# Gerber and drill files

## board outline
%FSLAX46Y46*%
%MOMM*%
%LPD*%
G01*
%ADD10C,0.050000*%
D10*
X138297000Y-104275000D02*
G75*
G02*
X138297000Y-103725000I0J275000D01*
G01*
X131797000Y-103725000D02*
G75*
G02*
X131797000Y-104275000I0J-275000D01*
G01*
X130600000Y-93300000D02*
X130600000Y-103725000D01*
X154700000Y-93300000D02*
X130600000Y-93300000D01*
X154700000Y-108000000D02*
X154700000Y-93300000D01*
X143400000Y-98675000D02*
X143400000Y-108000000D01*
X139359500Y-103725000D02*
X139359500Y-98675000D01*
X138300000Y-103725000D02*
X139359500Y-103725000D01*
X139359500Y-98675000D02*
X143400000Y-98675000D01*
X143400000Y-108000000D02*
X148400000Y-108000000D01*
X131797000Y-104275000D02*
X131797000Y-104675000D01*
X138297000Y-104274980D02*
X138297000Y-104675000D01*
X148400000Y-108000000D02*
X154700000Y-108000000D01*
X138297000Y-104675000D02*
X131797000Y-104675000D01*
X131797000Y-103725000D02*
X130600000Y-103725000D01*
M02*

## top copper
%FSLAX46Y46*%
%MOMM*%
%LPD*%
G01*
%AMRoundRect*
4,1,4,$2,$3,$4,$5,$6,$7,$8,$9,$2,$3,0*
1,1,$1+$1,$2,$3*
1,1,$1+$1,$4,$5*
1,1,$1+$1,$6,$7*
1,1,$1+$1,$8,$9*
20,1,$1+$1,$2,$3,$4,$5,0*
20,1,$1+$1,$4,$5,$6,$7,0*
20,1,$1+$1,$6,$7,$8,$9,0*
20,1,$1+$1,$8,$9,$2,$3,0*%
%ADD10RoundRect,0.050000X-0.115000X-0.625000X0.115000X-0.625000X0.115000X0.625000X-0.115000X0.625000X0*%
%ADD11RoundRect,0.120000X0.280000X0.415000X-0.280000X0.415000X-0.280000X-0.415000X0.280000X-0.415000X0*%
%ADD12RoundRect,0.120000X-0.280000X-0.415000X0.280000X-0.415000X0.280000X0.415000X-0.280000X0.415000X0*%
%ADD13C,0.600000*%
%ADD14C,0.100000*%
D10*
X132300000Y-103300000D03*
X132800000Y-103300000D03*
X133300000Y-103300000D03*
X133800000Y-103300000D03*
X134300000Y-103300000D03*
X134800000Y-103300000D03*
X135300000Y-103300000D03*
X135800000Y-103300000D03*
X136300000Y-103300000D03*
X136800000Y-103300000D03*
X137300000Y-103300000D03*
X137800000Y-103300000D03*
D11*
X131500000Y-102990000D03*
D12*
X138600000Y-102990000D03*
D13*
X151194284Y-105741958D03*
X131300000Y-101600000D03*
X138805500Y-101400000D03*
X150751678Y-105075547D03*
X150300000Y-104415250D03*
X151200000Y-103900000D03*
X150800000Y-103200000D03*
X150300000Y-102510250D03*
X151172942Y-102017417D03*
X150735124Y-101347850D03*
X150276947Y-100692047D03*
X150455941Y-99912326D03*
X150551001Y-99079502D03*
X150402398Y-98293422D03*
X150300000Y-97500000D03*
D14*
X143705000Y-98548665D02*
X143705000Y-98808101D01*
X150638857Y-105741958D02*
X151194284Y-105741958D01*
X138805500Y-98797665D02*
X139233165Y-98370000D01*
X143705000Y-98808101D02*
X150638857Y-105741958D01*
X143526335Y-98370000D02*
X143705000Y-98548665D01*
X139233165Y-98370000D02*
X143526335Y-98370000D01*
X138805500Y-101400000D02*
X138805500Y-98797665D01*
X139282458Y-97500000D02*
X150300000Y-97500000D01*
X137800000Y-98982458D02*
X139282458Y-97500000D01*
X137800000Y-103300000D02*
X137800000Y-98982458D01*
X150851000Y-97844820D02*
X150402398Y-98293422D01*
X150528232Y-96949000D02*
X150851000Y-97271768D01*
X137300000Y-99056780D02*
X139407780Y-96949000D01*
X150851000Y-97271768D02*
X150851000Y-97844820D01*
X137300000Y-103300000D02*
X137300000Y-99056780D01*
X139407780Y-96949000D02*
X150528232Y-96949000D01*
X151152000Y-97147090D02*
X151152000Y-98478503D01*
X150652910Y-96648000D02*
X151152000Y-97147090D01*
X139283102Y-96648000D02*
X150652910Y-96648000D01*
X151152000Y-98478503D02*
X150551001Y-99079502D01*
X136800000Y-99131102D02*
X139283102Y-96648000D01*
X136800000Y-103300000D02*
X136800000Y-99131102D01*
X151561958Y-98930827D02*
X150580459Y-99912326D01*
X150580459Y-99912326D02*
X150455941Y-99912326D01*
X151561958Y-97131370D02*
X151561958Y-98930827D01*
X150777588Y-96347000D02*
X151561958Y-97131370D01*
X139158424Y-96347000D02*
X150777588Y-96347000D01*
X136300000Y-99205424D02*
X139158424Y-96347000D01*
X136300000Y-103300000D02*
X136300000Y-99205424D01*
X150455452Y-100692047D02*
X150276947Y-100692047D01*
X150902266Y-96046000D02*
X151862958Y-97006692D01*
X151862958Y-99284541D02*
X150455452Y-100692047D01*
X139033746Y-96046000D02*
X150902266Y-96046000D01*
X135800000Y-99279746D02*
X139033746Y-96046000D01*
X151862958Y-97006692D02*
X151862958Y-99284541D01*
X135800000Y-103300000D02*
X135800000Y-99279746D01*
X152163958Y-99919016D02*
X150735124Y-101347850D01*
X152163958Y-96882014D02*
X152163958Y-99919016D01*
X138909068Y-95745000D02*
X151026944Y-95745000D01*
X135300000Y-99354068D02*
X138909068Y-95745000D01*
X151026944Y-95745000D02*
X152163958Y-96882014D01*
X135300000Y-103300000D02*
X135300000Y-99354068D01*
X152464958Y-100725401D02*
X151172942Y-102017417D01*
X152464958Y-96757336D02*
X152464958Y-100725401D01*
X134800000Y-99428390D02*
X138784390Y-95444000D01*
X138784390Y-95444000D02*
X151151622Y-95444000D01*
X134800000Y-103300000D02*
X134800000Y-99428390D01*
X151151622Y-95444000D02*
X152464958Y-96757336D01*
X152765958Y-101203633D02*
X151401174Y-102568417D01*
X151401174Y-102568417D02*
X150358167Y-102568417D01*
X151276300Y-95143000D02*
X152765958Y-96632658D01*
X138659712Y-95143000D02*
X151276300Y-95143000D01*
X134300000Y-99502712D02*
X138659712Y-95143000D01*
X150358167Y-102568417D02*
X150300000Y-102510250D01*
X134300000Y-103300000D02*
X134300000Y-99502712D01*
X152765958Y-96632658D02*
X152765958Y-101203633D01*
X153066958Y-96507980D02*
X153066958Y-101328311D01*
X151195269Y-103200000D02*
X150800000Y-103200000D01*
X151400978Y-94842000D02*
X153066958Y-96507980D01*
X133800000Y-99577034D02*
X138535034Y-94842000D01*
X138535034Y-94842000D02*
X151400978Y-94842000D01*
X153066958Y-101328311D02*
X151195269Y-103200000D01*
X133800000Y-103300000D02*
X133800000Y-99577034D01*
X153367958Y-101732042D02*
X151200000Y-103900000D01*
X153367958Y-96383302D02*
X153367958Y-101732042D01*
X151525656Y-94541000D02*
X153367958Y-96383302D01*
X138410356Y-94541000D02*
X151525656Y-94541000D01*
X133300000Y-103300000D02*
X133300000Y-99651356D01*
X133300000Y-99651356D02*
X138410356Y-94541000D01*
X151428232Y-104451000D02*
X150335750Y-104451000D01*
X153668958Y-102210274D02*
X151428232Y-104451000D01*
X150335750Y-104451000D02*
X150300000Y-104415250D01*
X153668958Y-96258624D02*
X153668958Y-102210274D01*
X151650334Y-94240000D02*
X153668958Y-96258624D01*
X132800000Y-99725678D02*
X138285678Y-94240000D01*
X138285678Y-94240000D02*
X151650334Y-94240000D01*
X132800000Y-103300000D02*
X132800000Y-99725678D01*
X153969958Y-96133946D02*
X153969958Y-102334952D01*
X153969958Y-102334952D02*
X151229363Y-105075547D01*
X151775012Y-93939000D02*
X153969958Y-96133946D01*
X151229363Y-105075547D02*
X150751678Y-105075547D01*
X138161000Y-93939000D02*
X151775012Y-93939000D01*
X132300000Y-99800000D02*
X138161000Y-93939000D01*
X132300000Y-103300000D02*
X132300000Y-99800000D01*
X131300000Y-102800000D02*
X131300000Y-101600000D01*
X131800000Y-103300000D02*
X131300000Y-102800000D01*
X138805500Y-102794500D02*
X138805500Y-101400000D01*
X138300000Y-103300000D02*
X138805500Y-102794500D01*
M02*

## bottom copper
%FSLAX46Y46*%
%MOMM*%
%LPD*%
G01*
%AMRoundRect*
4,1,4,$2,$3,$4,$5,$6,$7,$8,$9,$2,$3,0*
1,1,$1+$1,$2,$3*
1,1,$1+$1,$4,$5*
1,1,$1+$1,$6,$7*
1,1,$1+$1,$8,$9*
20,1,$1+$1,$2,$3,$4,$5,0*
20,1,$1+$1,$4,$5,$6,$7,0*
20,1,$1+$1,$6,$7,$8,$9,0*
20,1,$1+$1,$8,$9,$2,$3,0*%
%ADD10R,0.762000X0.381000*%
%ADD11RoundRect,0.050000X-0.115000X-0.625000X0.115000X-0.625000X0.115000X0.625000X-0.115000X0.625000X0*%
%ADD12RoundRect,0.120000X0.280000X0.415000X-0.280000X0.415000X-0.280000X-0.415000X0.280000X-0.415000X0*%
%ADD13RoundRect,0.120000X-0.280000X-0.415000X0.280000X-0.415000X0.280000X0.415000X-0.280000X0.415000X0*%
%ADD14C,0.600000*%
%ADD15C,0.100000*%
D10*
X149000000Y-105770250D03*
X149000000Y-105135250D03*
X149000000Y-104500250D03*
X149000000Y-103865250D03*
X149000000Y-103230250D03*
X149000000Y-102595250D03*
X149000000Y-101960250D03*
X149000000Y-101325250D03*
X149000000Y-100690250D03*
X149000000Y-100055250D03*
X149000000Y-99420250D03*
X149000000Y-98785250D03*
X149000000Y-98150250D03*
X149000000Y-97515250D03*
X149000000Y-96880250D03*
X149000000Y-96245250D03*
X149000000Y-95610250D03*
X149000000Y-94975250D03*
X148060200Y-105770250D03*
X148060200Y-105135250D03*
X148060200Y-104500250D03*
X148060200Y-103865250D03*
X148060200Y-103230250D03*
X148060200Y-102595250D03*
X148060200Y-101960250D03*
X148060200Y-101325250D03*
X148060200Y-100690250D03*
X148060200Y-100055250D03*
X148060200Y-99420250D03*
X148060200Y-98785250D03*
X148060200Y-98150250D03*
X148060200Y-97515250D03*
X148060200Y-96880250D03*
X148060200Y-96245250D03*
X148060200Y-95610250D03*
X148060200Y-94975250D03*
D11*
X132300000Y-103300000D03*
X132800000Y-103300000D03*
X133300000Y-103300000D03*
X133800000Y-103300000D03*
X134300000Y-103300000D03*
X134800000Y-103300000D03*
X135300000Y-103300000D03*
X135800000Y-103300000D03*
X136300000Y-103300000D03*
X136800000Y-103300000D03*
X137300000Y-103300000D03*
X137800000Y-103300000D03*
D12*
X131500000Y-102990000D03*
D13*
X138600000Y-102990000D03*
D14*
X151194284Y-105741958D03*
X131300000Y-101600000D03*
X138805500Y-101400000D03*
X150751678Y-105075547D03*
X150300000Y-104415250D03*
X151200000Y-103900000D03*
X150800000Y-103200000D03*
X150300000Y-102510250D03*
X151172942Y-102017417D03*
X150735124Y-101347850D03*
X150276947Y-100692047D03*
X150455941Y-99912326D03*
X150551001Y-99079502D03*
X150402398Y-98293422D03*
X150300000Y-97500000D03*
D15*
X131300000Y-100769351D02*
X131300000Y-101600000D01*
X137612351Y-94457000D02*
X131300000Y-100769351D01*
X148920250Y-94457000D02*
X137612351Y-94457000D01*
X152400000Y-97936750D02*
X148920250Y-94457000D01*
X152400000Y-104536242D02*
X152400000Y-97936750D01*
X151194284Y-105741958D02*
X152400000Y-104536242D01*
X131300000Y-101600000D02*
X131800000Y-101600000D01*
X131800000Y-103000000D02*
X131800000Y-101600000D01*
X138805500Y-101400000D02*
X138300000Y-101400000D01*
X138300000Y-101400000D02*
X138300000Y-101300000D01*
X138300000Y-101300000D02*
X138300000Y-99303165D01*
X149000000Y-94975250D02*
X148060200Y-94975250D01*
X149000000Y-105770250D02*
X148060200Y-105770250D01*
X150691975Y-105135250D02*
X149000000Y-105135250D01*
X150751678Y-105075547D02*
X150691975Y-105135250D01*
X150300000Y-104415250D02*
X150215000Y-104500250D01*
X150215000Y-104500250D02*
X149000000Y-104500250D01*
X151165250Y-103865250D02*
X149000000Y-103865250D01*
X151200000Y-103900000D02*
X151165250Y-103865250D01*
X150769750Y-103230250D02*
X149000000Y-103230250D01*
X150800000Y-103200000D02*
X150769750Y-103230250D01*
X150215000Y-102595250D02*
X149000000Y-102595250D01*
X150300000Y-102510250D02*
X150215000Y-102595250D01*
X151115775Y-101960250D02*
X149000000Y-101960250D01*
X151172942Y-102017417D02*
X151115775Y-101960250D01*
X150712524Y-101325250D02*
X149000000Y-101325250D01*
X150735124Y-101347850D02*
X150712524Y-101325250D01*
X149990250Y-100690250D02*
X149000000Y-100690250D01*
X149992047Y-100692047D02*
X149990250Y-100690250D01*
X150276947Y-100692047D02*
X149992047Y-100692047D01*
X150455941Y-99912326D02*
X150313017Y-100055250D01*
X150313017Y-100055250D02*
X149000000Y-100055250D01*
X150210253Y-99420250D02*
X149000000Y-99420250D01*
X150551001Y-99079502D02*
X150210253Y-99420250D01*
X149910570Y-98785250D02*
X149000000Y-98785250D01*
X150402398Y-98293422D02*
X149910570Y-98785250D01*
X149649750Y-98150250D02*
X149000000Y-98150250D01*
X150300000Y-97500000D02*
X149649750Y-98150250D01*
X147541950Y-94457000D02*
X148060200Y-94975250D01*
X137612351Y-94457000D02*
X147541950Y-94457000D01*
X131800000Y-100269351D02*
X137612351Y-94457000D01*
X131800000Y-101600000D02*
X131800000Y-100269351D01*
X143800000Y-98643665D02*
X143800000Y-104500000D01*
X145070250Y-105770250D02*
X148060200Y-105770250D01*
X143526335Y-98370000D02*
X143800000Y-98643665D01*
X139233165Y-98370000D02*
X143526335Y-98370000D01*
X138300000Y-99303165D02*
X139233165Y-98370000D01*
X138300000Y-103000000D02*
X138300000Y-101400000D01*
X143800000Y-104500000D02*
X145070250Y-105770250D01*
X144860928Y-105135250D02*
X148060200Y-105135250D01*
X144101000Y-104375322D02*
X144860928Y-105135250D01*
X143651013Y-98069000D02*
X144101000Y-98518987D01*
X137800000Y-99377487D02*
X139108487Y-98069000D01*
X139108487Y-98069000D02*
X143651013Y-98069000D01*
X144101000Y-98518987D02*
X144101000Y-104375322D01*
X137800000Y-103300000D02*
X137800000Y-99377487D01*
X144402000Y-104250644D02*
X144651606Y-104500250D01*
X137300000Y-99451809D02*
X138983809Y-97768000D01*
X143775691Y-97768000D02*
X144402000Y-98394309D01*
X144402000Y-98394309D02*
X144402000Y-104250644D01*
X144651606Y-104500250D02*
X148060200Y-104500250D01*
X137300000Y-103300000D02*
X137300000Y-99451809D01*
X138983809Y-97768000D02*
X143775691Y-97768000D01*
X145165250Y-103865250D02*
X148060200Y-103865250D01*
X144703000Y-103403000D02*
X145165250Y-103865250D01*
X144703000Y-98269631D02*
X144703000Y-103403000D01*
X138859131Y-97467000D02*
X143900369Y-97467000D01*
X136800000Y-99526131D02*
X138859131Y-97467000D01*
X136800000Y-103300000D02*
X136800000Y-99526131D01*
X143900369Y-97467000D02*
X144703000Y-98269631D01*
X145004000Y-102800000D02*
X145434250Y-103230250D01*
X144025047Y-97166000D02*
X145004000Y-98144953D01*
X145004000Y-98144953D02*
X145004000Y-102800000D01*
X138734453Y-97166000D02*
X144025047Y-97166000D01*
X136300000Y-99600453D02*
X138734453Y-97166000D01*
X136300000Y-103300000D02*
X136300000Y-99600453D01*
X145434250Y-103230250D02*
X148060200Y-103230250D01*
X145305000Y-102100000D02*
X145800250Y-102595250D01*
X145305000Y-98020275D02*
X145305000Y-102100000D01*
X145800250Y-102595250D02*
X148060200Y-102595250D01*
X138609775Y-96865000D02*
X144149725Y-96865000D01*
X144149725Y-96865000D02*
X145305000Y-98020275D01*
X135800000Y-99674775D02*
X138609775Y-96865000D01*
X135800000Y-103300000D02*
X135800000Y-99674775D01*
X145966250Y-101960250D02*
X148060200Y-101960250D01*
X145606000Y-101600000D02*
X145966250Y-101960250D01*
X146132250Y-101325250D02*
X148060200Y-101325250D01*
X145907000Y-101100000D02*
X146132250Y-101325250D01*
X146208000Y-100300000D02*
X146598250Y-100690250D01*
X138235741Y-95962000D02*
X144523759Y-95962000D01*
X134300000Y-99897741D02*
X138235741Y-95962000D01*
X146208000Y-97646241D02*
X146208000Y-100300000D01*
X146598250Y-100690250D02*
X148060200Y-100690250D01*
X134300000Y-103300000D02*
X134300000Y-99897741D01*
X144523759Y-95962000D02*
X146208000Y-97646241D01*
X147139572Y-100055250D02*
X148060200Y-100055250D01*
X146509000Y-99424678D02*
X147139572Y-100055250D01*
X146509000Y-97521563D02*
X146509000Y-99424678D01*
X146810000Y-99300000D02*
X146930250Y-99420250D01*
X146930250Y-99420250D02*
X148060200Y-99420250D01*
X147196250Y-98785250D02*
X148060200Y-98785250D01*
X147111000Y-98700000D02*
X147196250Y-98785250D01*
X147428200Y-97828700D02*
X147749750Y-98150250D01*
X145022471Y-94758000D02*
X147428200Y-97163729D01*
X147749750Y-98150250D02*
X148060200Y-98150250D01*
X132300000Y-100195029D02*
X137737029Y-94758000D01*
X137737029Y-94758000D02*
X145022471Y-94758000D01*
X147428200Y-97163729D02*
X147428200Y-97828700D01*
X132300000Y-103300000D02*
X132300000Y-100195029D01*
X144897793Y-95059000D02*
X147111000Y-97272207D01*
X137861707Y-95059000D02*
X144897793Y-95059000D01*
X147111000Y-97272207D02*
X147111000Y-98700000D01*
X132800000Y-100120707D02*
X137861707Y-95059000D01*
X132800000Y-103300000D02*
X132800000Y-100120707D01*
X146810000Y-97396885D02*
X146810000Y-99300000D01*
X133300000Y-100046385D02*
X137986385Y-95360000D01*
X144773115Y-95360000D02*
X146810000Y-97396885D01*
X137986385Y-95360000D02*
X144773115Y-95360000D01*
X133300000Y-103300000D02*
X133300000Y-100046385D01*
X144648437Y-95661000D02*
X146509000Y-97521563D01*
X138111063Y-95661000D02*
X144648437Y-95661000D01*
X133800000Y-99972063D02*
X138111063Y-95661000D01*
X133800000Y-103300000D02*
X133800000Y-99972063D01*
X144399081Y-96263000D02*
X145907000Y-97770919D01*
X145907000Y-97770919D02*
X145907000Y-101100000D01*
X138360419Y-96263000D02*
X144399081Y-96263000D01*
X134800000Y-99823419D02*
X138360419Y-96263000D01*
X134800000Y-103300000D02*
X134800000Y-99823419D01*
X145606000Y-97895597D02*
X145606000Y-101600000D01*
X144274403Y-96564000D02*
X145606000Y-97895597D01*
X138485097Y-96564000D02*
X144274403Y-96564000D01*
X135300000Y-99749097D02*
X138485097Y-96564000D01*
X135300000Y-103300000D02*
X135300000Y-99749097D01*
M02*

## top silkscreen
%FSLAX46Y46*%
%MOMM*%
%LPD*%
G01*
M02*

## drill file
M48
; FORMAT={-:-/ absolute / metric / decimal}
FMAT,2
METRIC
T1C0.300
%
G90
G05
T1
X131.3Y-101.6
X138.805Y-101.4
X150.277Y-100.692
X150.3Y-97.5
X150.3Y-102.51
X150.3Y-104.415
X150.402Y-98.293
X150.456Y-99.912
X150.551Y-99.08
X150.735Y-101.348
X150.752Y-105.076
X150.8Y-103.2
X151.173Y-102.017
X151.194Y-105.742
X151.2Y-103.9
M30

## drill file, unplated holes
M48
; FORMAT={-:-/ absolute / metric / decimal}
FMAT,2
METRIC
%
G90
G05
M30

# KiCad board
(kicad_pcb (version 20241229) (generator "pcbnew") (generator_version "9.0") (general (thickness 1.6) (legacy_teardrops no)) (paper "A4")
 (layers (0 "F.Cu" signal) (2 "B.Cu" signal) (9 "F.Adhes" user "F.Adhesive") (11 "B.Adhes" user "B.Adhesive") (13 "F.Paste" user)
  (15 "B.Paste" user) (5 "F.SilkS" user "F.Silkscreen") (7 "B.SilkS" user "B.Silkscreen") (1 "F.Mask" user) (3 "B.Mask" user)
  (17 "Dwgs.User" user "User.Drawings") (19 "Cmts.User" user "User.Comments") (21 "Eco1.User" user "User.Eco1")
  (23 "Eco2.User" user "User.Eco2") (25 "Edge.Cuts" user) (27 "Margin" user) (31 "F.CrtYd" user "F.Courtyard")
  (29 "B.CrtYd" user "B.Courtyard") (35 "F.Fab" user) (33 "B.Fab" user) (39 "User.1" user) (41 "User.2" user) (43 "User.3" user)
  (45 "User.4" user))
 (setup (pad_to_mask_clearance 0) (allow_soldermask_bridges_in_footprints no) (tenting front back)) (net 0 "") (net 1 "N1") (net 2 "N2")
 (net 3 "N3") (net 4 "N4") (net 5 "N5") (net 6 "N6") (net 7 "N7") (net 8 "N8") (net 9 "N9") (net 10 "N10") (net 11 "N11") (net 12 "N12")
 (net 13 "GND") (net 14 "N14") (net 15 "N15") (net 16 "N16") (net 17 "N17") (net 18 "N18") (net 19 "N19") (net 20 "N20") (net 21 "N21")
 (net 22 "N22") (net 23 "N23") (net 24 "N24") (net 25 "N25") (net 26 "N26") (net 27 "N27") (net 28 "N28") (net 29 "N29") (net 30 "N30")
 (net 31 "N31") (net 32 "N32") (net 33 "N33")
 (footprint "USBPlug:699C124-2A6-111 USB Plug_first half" (layer "F.Cu") (at 134.8 100.3)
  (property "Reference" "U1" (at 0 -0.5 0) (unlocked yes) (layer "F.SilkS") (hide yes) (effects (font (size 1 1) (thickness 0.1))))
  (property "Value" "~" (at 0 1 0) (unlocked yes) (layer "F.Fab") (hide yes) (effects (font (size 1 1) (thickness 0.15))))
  (pad "0" smd roundrect (at -2.5 3) (size 0.33 1.35) (layers "F.Cu" "F.Mask" "F.Paste") (roundrect_rratio 0.1515151515) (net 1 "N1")
   (thermal_bridge_angle 45))
  (pad "1" smd roundrect (at -2 3) (size 0.33 1.35) (layers "F.Cu" "F.Mask" "F.Paste") (roundrect_rratio 0.1515151515) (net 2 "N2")
   (thermal_bridge_angle 45))
  (pad "2" smd roundrect (at -1.5 3) (size 0.33 1.35) (layers "F.Cu" "F.Mask" "F.Paste") (roundrect_rratio 0.1515151515) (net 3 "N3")
   (thermal_bridge_angle 45))
  (pad "3" smd roundrect (at -1 3) (size 0.33 1.35) (layers "F.Cu" "F.Mask" "F.Paste") (roundrect_rratio 0.1515151515) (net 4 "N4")
   (thermal_bridge_angle 45))
  (pad "4" smd roundrect (at -0.5 3) (size 0.33 1.35) (layers "F.Cu" "F.Mask" "F.Paste") (roundrect_rratio 0.1515151515) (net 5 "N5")
   (thermal_bridge_angle 45))
  (pad "5" smd roundrect (at 0 3) (size 0.33 1.35) (layers "F.Cu" "F.Mask" "F.Paste") (roundrect_rratio 0.1515151515) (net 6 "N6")
   (thermal_bridge_angle 45))
  (pad "6" smd roundrect (at 0.5 3) (size 0.33 1.35) (layers "F.Cu" "F.Mask" "F.Paste") (roundrect_rratio 0.1515151515) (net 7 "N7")
   (thermal_bridge_angle 45))
  (pad "7" smd roundrect (at 1 3) (size 0.33 1.35) (layers "F.Cu" "F.Mask" "F.Paste") (roundrect_rratio 0.1515151515) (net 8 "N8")
   (thermal_bridge_angle 45))
  (pad "8" smd roundrect (at 1.5 3) (size 0.33 1.35) (layers "F.Cu" "F.Mask" "F.Paste") (roundrect_rratio 0.1515151515) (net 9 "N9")
   (thermal_bridge_angle 45))
  (pad "9" smd roundrect (at 2 3) (size 0.33 1.35) (layers "F.Cu" "F.Mask" "F.Paste") (roundrect_rratio 0.1515151515) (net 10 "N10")
   (thermal_bridge_angle 45))
  (pad "10" smd roundrect (at 2.5 3) (size 0.33 1.35) (layers "F.Cu" "F.Mask" "F.Paste") (roundrect_rratio 0.1515151515) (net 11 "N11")
   (thermal_bridge_angle 45))
  (pad "11" smd roundrect (at 3 3) (size 0.33 1.35) (layers "F.Cu" "F.Mask" "F.Paste") (roundrect_rratio 0.1515151515) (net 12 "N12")
   (thermal_bridge_angle 45))
  (pad "24" smd roundrect (at -3 3 180) (size 0.8 1.07) (drill (offset 0.3 0.31)) (layers "F.Cu" "F.Mask" "F.Paste") (roundrect_rratio 0.15)
   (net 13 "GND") (thermal_bridge_angle 45))
  (pad "25" smd roundrect (at 3.5 3) (size 0.8 1.07) (drill (offset 0.3 -0.31)) (layers "F.Cu" "F.Mask" "F.Paste") (roundrect_rratio 0.15)
   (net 13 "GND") (thermal_bridge_angle 45)))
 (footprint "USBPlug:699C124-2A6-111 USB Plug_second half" (layer "B.Cu") (at 134.8 106.3)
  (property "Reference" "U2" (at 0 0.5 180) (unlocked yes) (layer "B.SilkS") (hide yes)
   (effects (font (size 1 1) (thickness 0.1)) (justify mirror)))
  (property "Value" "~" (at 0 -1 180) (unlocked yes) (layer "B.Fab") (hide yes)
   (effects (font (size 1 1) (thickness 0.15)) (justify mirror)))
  (pad "12" smd roundrect (at -2.5 -3) (size 0.33 1.35) (layers "B.Cu" "B.Mask" "B.Paste") (roundrect_rratio 0.1515151515) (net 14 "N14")
   (thermal_bridge_angle 45))
  (pad "13" smd roundrect (at -2 -3) (size 0.33 1.35) (layers "B.Cu" "B.Mask" "B.Paste") (roundrect_rratio 0.1515151515) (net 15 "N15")
   (thermal_bridge_angle 45))
  (pad "14" smd roundrect (at -1.5 -3) (size 0.33 1.35) (layers "B.Cu" "B.Mask" "B.Paste") (roundrect_rratio 0.1515151515) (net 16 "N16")
   (thermal_bridge_angle 45))
  (pad "15" smd roundrect (at -1 -3) (size 0.33 1.35) (layers "B.Cu" "B.Mask" "B.Paste") (roundrect_rratio 0.1515151515) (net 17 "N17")
   (thermal_bridge_angle 45))
  (pad "16" smd roundrect (at -0.5 -3) (size 0.33 1.35) (layers "B.Cu" "B.Mask" "B.Paste") (roundrect_rratio 0.1515151515) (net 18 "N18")
   (thermal_bridge_angle 45))
  (pad "17" smd roundrect (at 0 -3) (size 0.33 1.35) (layers "B.Cu" "B.Mask" "B.Paste") (roundrect_rratio 0.1515151515) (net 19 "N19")
   (thermal_bridge_angle 45))
  (pad "18" smd roundrect (at 0.5 -3) (size 0.33 1.35) (layers "B.Cu" "B.Mask" "B.Paste") (roundrect_rratio 0.1515151515) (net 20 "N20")
   (thermal_bridge_angle 45))
  (pad "19" smd roundrect (at 1 -3) (size 0.33 1.35) (layers "B.Cu" "B.Mask" "B.Paste") (roundrect_rratio 0.1515151515) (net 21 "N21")
   (thermal_bridge_angle 45))
  (pad "20" smd roundrect (at 1.5 -3) (size 0.33 1.35) (layers "B.Cu" "B.Mask" "B.Paste") (roundrect_rratio 0.1515151515) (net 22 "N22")
   (thermal_bridge_angle 45))
  (pad "21" smd roundrect (at 2 -3) (size 0.33 1.35) (layers "B.Cu" "B.Mask" "B.Paste") (roundrect_rratio 0.1515151515) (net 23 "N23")
   (thermal_bridge_angle 45))
  (pad "22" smd roundrect (at 2.5 -3) (size 0.33 1.35) (layers "B.Cu" "B.Mask" "B.Paste") (roundrect_rratio 0.1515151515) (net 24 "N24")
   (thermal_bridge_angle 45))
  (pad "23" smd roundrect (at 3 -3) (size 0.33 1.35) (layers "B.Cu" "B.Mask" "B.Paste") (roundrect_rratio 0.1515151515) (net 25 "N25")
   (thermal_bridge_angle 45))
  (pad "26" smd roundrect (at -3 -3.3 180) (size 0.8 1.07) (drill (offset 0.3 0.01)) (layers "B.Cu" "B.Mask" "B.Paste")
   (roundrect_rratio 0.15) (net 13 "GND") (thermal_bridge_angle 45))
  (pad "27" smd roundrect (at 3.5 -3.3) (size 0.8 1.07) (drill (offset 0.3 -0.01)) (layers "B.Cu" "B.Mask" "B.Paste")
   (roundrect_rratio 0.15) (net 13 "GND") (thermal_bridge_angle 45)))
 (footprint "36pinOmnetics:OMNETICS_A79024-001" (layer "B.Cu") (at 148.5301 100.37275 -90)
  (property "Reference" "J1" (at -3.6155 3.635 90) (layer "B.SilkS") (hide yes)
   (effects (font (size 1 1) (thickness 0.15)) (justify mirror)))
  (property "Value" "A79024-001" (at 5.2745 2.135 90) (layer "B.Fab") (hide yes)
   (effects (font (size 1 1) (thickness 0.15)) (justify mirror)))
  (pad "1" smd rect (at 5.3975 -0.4699 270) (size 0.381 0.762) (layers "B.Cu" "B.Mask" "B.Paste") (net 13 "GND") (solder_mask_margin 0.102))
  (pad "2" smd rect (at 4.7625 -0.4699 270) (size 0.381 0.762) (layers "B.Cu" "B.Mask" "B.Paste") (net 1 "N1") (solder_mask_margin 0.102))
  (pad "3" smd rect (at 4.1275 -0.4699 270) (size 0.381 0.762) (layers "B.Cu" "B.Mask" "B.Paste") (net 2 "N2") (solder_mask_margin 0.102))
  (pad "4" smd rect (at 3.4925 -0.4699 270) (size 0.381 0.762) (layers "B.Cu" "B.Mask" "B.Paste") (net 3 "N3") (solder_mask_margin 0.102))
  (pad "5" smd rect (at 2.8575 -0.4699 270) (size 0.381 0.762) (layers "B.Cu" "B.Mask" "B.Paste") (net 4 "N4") (solder_mask_margin 0.102))
  (pad "6" smd rect (at 2.2225 -0.4699 270) (size 0.381 0.762) (layers "B.Cu" "B.Mask" "B.Paste") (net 5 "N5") (solder_mask_margin 0.102))
  (pad "7" smd rect (at 1.5875 -0.4699 270) (size 0.381 0.762) (layers "B.Cu" "B.Mask" "B.Paste") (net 6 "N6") (solder_mask_margin 0.102))
  (pad "8" smd rect (at 0.9525 -0.4699 270) (size 0.381 0.762) (layers "B.Cu" "B.Mask" "B.Paste") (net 7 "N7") (solder_mask_margin 0.102))
  (pad "9" smd rect (at 0.3175 -0.4699 270) (size 0.381 0.762) (layers "B.Cu" "B.Mask" "B.Paste") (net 8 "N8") (solder_mask_margin 0.102))
  (pad "10" smd rect (at -0.3175 -0.4699 270) (size 0.381 0.762) (layers "B.Cu" "B.Mask" "B.Paste") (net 9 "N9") (solder_mask_margin 0.102))
  (pad "11" smd rect (at -0.9525 -0.4699 270) (size 0.381 0.762) (layers "B.Cu" "B.Mask" "B.Paste") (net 10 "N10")
   (solder_mask_margin 0.102))
  (pad "12" smd rect (at -1.5875 -0.4699 270) (size 0.381 0.762) (layers "B.Cu" "B.Mask" "B.Paste") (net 11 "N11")
   (solder_mask_margin 0.102))
  (pad "13" smd rect (at -2.2225 -0.4699 270) (size 0.381 0.762) (layers "B.Cu" "B.Mask" "B.Paste") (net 12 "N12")
   (solder_mask_margin 0.102))
  (pad "14" smd rect (at -2.8575 -0.4699 270) (size 0.381 0.762) (layers "B.Cu" "B.Mask" "B.Paste") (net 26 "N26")
   (solder_mask_margin 0.102))
  (pad "15" smd rect (at -3.4925 -0.4699 270) (size 0.381 0.762) (layers "B.Cu" "B.Mask" "B.Paste") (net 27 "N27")
   (solder_mask_margin 0.102))
  (pad "16" smd rect (at -4.1275 -0.4699 270) (size 0.381 0.762) (layers "B.Cu" "B.Mask" "B.Paste") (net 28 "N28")
   (solder_mask_margin 0.102))
  (pad "17" smd rect (at -4.7625 -0.4699 270) (size 0.381 0.762) (layers "B.Cu" "B.Mask" "B.Paste") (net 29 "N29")
   (solder_mask_margin 0.102))
  (pad "18" smd rect (at -5.3975 -0.4699 270) (size 0.381 0.762) (layers "B.Cu" "B.Mask" "B.Paste") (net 13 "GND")
   (solder_mask_margin 0.102))
  (pad "19" smd rect (at 5.3975 0.4699 270) (size 0.381 0.762) (layers "B.Cu" "B.Mask" "B.Paste") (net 13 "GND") (solder_mask_margin 0.102))
  (pad "20" smd rect (at 4.7625 0.4699 270) (size 0.381 0.762) (layers "B.Cu" "B.Mask" "B.Paste") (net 25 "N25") (solder_mask_margin 0.102))
  (pad "21" smd rect (at 4.1275 0.4699 270) (size 0.381 0.762) (layers "B.Cu" "B.Mask" "B.Paste") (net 24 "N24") (solder_mask_margin 0.102))
  (pad "22" smd rect (at 3.4925 0.4699 270) (size 0.381 0.762) (layers "B.Cu" "B.Mask" "B.Paste") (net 23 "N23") (solder_mask_margin 0.102))
  (pad "23" smd rect (at 2.8575 0.4699 270) (size 0.381 0.762) (layers "B.Cu" "B.Mask" "B.Paste") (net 22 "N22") (solder_mask_margin 0.102))
  (pad "24" smd rect (at 2.2225 0.4699 270) (size 0.381 0.762) (layers "B.Cu" "B.Mask" "B.Paste") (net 21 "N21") (solder_mask_margin 0.102))
  (pad "25" smd rect (at 1.5875 0.4699 270) (size 0.381 0.762) (layers "B.Cu" "B.Mask" "B.Paste") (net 20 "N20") (solder_mask_margin 0.102))
  (pad "26" smd rect (at 0.9525 0.4699 270) (size 0.381 0.762) (layers "B.Cu" "B.Mask" "B.Paste") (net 19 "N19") (solder_mask_margin 0.102))
  (pad "27" smd rect (at 0.3175 0.4699 270) (size 0.381 0.762) (layers "B.Cu" "B.Mask" "B.Paste") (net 18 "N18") (solder_mask_margin 0.102))
  (pad "28" smd rect (at -0.3175 0.4699 270) (size 0.381 0.762) (layers "B.Cu" "B.Mask" "B.Paste") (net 17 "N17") (solder_mask_margin 0.102))
  (pad "29" smd rect (at -0.9525 0.4699 270) (size 0.381 0.762) (layers "B.Cu" "B.Mask" "B.Paste") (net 16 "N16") (solder_mask_margin 0.102))
  (pad "30" smd rect (at -1.5875 0.4699 270) (size 0.381 0.762) (layers "B.Cu" "B.Mask" "B.Paste") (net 15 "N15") (solder_mask_margin 0.102))
  (pad "31" smd rect (at -2.2225 0.4699 270) (size 0.381 0.762) (layers "B.Cu" "B.Mask" "B.Paste") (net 14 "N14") (solder_mask_margin 0.102))
  (pad "32" smd rect (at -2.8575 0.4699 270) (size 0.381 0.762) (layers "B.Cu" "B.Mask" "B.Paste") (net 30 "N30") (solder_mask_margin 0.102))
  (pad "33" smd rect (at -3.4925 0.4699 270) (size 0.381 0.762) (layers "B.Cu" "B.Mask" "B.Paste") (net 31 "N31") (solder_mask_margin 0.102))
  (pad "34" smd rect (at -4.1275 0.4699 270) (size 0.381 0.762) (layers "B.Cu" "B.Mask" "B.Paste") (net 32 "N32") (solder_mask_margin 0.102))
  (pad "35" smd rect (at -4.7625 0.4699 270) (size 0.381 0.762) (layers "B.Cu" "B.Mask" "B.Paste") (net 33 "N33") (solder_mask_margin 0.102))
  (pad "36" smd rect (at -5.3975 0.4699 270) (size 0.381 0.762) (layers "B.Cu" "B.Mask" "B.Paste") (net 13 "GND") (solder_mask_margin 0.102)))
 (gr_line (start 154.7 93.3) (end 130.6 93.3) (stroke (width 0.05) (type default)) (layer "Edge.Cuts"))
 (gr_line (start 130.6 93.3) (end 130.6 103.725) (stroke (width 0.05) (type default)) (layer "Edge.Cuts"))
 (gr_line (start 143.4 98.675) (end 143.4 108) (stroke (width 0.05) (type default)) (layer "Edge.Cuts"))
 (gr_line (start 139.3595 103.725) (end 139.3595 98.675) (stroke (width 0.05) (type default)) (layer "Edge.Cuts"))
 (gr_line (start 138.3 103.725) (end 139.3595 103.725) (stroke (width 0.05) (type default)) (layer "Edge.Cuts"))
 (gr_line (start 139.3595 98.675) (end 143.4 98.675) (stroke (width 0.05) (type default)) (layer "Edge.Cuts"))
 (gr_line (start 143.4 108) (end 148.4 108) (stroke (width 0.05) (type default)) (layer "Edge.Cuts"))
 (gr_line (start 131.797 104.275) (end 131.797 104.675) (stroke (width 0.05) (type default)) (layer "Edge.Cuts"))
 (gr_line (start 138.297 104.27498) (end 138.297 104.675) (stroke (width 0.05) (type default)) (layer "Edge.Cuts"))
 (gr_arc (start 131.797 103.725) (mid 132.072 104) (end 131.797 104.275) (stroke (width 0.05) (type default)) (layer "Edge.Cuts"))
 (gr_line (start 148.4 108) (end 154.7 108) (stroke (width 0.05) (type default)) (layer "Edge.Cuts"))
 (gr_arc (start 138.297 104.275) (mid 138.022 104) (end 138.297 103.725) (stroke (width 0.05) (type default)) (layer "Edge.Cuts"))
 (gr_line (start 154.7 108) (end 154.7 93.3) (stroke (width 0.05) (type default)) (layer "Edge.Cuts"))
 (gr_line (start 138.297 104.675) (end 131.797 104.675) (stroke (width 0.05) (type default)) (layer "Edge.Cuts"))
 (gr_line (start 131.797 103.725) (end 130.6 103.725) (stroke (width 0.05) (type default)) (layer "Edge.Cuts"))
 (segment (start 143.705 98.808101) (end 150.638857 105.741958) (width 0.1) (layer "F.Cu") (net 13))
 (segment (start 138.3 103.3) (end 138.8055 102.7945) (width 0.1) (layer "F.Cu") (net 13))
 (segment (start 131.3 102.8) (end 131.3 101.6) (width 0.1) (layer "F.Cu") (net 13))
 (segment (start 138.8055 101.4) (end 138.8055 98.797665) (width 0.1) (layer "F.Cu") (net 13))
 (segment (start 150.638857 105.741958) (end 151.194284 105.741958) (width 0.1) (layer "F.Cu") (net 13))
 (segment (start 138.8055 102.7945) (end 138.8055 101.4) (width 0.1) (layer "F.Cu") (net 13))
 (segment (start 138.8055 98.797665) (end 139.233165 98.37) (width 0.1) (layer "F.Cu") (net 13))
 (segment (start 139.233165 98.37) (end 143.526335 98.37) (width 0.1) (layer "F.Cu") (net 13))
 (segment (start 143.526335 98.37) (end 143.705 98.548665) (width 0.1) (layer "F.Cu") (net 13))
 (segment (start 143.705 98.548665) (end 143.705 98.808101) (width 0.1) (layer "F.Cu") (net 13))
 (segment (start 131.8 103.3) (end 131.3 102.8) (width 0.1) (layer "F.Cu") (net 13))
 (via (at 131.3 101.6) (size 0.6) (drill 0.3) (layers "F.Cu" "B.Cu") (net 13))
 (via (at 138.8055 101.4) (size 0.6) (drill 0.3) (layers "F.Cu" "B.Cu") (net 13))
 (via (at 151.194284 105.741958) (size 0.6) (drill 0.3) (layers "F.Cu" "B.Cu") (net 13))
 (segment (start 148.92025 94.457) (end 137.612351 94.457) (width 0.1) (layer "B.Cu") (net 13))
 (segment (start 145.07025 105.77025) (end 148.0602 105.77025) (width 0.1) (layer "B.Cu") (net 13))
 (segment (start 138.3 101.3) (end 138.3 99.303165) (width 0.1) (layer "B.Cu") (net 13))
 (segment (start 131.8 101.6) (end 131.8 100.269351) (width 0.1) (layer "B.Cu") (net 13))
 (segment (start 152.4 97.93675) (end 148.92025 94.457) (width 0.1) (layer "B.Cu") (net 13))
 (segment (start 143.526335 98.37) (end 143.8 98.643665) (width 0.1) (layer "B.Cu") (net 13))
 (segment (start 143.8 104.5) (end 145.07025 105.77025) (width 0.1) (layer "B.Cu") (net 13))
 (segment (start 139.233165 98.37) (end 143.526335 98.37) (width 0.1) (layer "B.Cu") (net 13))
 (segment (start 138.8055 101.4) (end 138.3 101.4) (width 0.1) (layer "B.Cu") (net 13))
 (segment (start 151.194284 105.741958) (end 152.4 104.536242) (width 0.1) (layer "B.Cu") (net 13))
 (segment (start 143.8 98.643665) (end 143.8 104.5) (width 0.1) (layer "B.Cu") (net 13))
 (segment (start 147.54195 94.457) (end 148.0602 94.97525) (width 0.1) (layer "B.Cu") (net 13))
 (segment (start 137.612351 94.457) (end 147.54195 94.457) (width 0.1) (layer "B.Cu") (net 13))
 (segment (start 149 105.77025) (end 148.0602 105.77025) (width 0.1) (layer "B.Cu") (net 13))
 (segment (start 138.3 103) (end 138.3 101.4) (width 0.1) (layer "B.Cu") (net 13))
 (segment (start 131.8 103) (end 131.8 101.6) (width 0.1) (layer "B.Cu") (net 13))
 (segment (start 131.3 100.769351) (end 131.3 101.6) (width 0.1) (layer "B.Cu") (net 13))
 (segment (start 137.612351 94.457) (end 131.3 100.769351) (width 0.1) (layer "B.Cu") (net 13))
 (segment (start 152.4 104.536242) (end 152.4 97.93675) (width 0.1) (layer "B.Cu") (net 13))
 (segment (start 149 94.97525) (end 148.0602 94.97525) (width 0.1) (layer "B.Cu") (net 13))
 (segment (start 131.3 101.6) (end 131.8 101.6) (width 0.1) (layer "B.Cu") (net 13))
 (segment (start 138.3 99.303165) (end 139.233165 98.37) (width 0.1) (layer "B.Cu") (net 13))
 (segment (start 138.3 101.4) (end 138.3 101.3) (width 0.1) (layer "B.Cu") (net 13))
 (segment (start 131.8 100.269351) (end 137.612351 94.457) (width 0.1) (layer "B.Cu") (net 13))
 (segment (start 133.3 99.651356) (end 138.410356 94.541) (width 0.1) (layer "F.Cu") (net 3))
 (segment (start 151.525656 94.541) (end 153.367958 96.383302) (width 0.1) (layer "F.Cu") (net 3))
 (segment (start 138.410356 94.541) (end 151.525656 94.541) (width 0.1) (layer "F.Cu") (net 3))
 (segment (start 153.367958 96.383302) (end 153.367958 101.732042) (width 0.1) (layer "F.Cu") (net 3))
 (segment (start 133.3 103.3) (end 133.3 99.651356) (width 0.1) (layer "F.Cu") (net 3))
 (segment (start 153.367958 101.732042) (end 151.2 103.9) (width 0.1) (layer "F.Cu") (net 3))
 (via (at 151.2 103.9) (size 0.6) (drill 0.3) (layers "F.Cu" "B.Cu") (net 3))
 (segment (start 151.2 103.9) (end 151.16525 103.86525) (width 0.1) (layer "B.Cu") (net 3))
 (segment (start 151.16525 103.86525) (end 149 103.86525) (width 0.1) (layer "B.Cu") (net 3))
 (segment (start 151.152 97.14709) (end 151.152 98.478503) (width 0.1) (layer "F.Cu") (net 10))
 (segment (start 136.8 103.3) (end 136.8 99.131102) (width 0.1) (layer "F.Cu") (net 10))
 (segment (start 139.283102 96.648) (end 150.65291 96.648) (width 0.1) (layer "F.Cu") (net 10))
 (segment (start 151.152 98.478503) (end 150.551001 99.079502) (width 0.1) (layer "F.Cu") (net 10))
 (segment (start 150.65291 96.648) (end 151.152 97.14709) (width 0.1) (layer "F.Cu") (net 10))
 (segment (start 136.8 99.131102) (end 139.283102 96.648) (width 0.1) (layer "F.Cu") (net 10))
 (via (at 150.551001 99.079502) (size 0.6) (drill 0.3) (layers "F.Cu" "B.Cu") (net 10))
 (segment (start 150.210253 99.42025) (end 149 99.42025) (width 0.1) (layer "B.Cu") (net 10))
 (segment (start 150.551001 99.079502) (end 150.210253 99.42025) (width 0.1) (layer "B.Cu") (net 10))
 (segment (start 152.765958 101.203633) (end 151.401174 102.568417) (width 0.1) (layer "F.Cu") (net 5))
 (segment (start 150.358167 102.568417) (end 150.3 102.51025) (width 0.1) (layer "F.Cu") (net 5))
 (segment (start 134.3 103.3) (end 134.3 99.502712) (width 0.1) (layer "F.Cu") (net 5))
 (segment (start 152.765958 96.632658) (end 152.765958 101.203633) (width 0.1) (layer "F.Cu") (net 5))
 (segment (start 134.3 99.502712) (end 138.659712 95.143) (width 0.1) (layer "F.Cu") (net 5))
 (segment (start 151.401174 102.568417) (end 150.358167 102.568417) (width 0.1) (layer "F.Cu") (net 5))
 (segment (start 151.2763 95.143) (end 152.765958 96.632658) (width 0.1) (layer "F.Cu") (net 5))
 (segment (start 138.659712 95.143) (end 151.2763 95.143) (width 0.1) (layer "F.Cu") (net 5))
 (via (at 150.3 102.51025) (size 0.6) (drill 0.3) (layers "F.Cu" "B.Cu") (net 5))
 (segment (start 150.3 102.51025) (end 150.215 102.59525) (width 0.1) (layer "B.Cu") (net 5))
 (segment (start 150.215 102.59525) (end 149 102.59525) (width 0.1) (layer "B.Cu") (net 5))
 (segment (start 139.033746 96.046) (end 150.902266 96.046) (width 0.1) (layer "F.Cu") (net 8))
 (segment (start 135.8 103.3) (end 135.8 99.279746) (width 0.1) (layer "F.Cu") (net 8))
 (segment (start 150.902266 96.046) (end 151.862958 97.006692) (width 0.1) (layer "F.Cu") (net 8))
 (segment (start 150.455452 100.692047) (end 150.276947 100.692047) (width 0.1) (layer "F.Cu") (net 8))
 (segment (start 135.8 99.279746) (end 139.033746 96.046) (width 0.1) (layer "F.Cu") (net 8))
 (segment (start 151.862958 97.006692) (end 151.862958 99.284541) (width 0.1) (layer "F.Cu") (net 8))
 (segment (start 151.862958 99.284541) (end 150.455452 100.692047) (width 0.1) (layer "F.Cu") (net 8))
 (via (at 150.276947 100.692047) (size 0.6) (drill 0.3) (layers "F.Cu" "B.Cu") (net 8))
 (segment (start 149.992047 100.692047) (end 149.99025 100.69025) (width 0.1) (layer "B.Cu") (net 8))
 (segment (start 149.99025 100.69025) (end 149 100.69025) (width 0.1) (layer "B.Cu") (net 8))
 (segment (start 150.276947 100.692047) (end 149.992047 100.692047) (width 0.1) (layer "B.Cu") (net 8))
 (segment (start 145.305 98.020275) (end 145.305 102.1) (width 0.1) (layer "B.Cu") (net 21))
 (segment (start 145.80025 102.59525) (end 148.0602 102.59525) (width 0.1) (layer "B.Cu") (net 21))
 (segment (start 135.8 99.674775) (end 138.609775 96.865) (width 0.1) (layer "B.Cu") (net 21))
 (segment (start 145.305 102.1) (end 145.80025 102.59525) (width 0.1) (layer "B.Cu") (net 21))
 (segment (start 144.149725 96.865) (end 145.305 98.020275) (width 0.1) (layer "B.Cu") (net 21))
 (segment (start 135.8 103.3) (end 135.8 99.674775) (width 0.1) (layer "B.Cu") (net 21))
 (segment (start 138.609775 96.865) (end 144.149725 96.865) (width 0.1) (layer "B.Cu") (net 21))
 (segment (start 145.004 102.8) (end 145.43425 103.23025) (width 0.1) (layer "B.Cu") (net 22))
 (segment (start 136.3 103.3) (end 136.3 99.600453) (width 0.1) (layer "B.Cu") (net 22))
 (segment (start 138.734453 97.166) (end 144.025047 97.166) (width 0.1) (layer "B.Cu") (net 22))
 (segment (start 136.3 99.600453) (end 138.734453 97.166) (width 0.1) (layer "B.Cu") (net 22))
 (segment (start 144.025047 97.166) (end 145.004 98.144953) (width 0.1) (layer "B.Cu") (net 22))
 (segment (start 145.43425 103.23025) (end 148.0602 103.23025) (width 0.1) (layer "B.Cu") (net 22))
 (segment (start 145.004 98.144953) (end 145.004 102.8) (width 0.1) (layer "B.Cu") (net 22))
 (segment (start 137.3 99.05678) (end 139.40778 96.949) (width 0.1) (layer "F.Cu") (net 11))
 (segment (start 150.528232 96.949) (end 150.851 97.271768) (width 0.1) (layer "F.Cu") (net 11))
 (segment (start 139.40778 96.949) (end 150.528232 96.949) (width 0.1) (layer "F.Cu") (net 11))
 (segment (start 150.851 97.271768) (end 150.851 97.84482) (width 0.1) (layer "F.Cu") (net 11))
 (segment (start 150.851 97.84482) (end 150.402398 98.293422) (width 0.1) (layer "F.Cu") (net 11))
 (segment (start 137.3 103.3) (end 137.3 99.05678) (width 0.1) (layer "F.Cu") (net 11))
 (via (at 150.402398 98.293422) (size 0.6) (drill 0.3) (layers "F.Cu" "B.Cu") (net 11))
 (segment (start 150.402398 98.293422) (end 149.91057 98.78525) (width 0.1) (layer "B.Cu") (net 11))
 (segment (start 149.91057 98.78525) (end 149 98.78525) (width 0.1) (layer "B.Cu") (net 11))
 (segment (start 152.464958 96.757336) (end 152.464958 100.725401) (width 0.1) (layer "F.Cu") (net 6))
 (segment (start 151.151622 95.444) (end 152.464958 96.757336) (width 0.1) (layer "F.Cu") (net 6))
 (segment (start 138.78439 95.444) (end 151.151622 95.444) (width 0.1) (layer "F.Cu") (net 6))
 (segment (start 134.8 99.42839) (end 138.78439 95.444) (width 0.1) (layer "F.Cu") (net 6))
 (segment (start 134.8 103.3) (end 134.8 99.42839) (width 0.1) (layer "F.Cu") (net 6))
 (segment (start 152.464958 100.725401) (end 151.172942 102.017417) (width 0.1) (layer "F.Cu") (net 6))
 (via (at 151.172942 102.017417) (size 0.6) (drill 0.3) (layers "F.Cu" "B.Cu") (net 6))
 (segment (start 151.172942 102.017417) (end 151.115775 101.96025) (width 0.1) (layer "B.Cu") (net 6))
 (segment (start 151.115775 101.96025) (end 149 101.96025) (width 0.1) (layer "B.Cu") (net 6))
 (segment (start 150.580459 99.912326) (end 150.455941 99.912326) (width 0.1) (layer "F.Cu") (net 9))
 (segment (start 151.561958 98.930827) (end 150.580459 99.912326) (width 0.1) (layer "F.Cu") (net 9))
 (segment (start 139.158424 96.347) (end 150.777588 96.347) (width 0.1) (layer "F.Cu") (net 9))
 (segment (start 136.3 99.205424) (end 139.158424 96.347) (width 0.1) (layer "F.Cu") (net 9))
 (segment (start 136.3 103.3) (end 136.3 99.205424) (width 0.1) (layer "F.Cu") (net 9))
 (segment (start 151.561958 97.13137) (end 151.561958 98.930827) (width 0.1) (layer "F.Cu") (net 9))
 (segment (start 150.777588 96.347) (end 151.561958 97.13137) (width 0.1) (layer "F.Cu") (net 9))
 (via (at 150.455941 99.912326) (size 0.6) (drill 0.3) (layers "F.Cu" "B.Cu") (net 9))
 (segment (start 150.455941 99.912326) (end 150.313017 100.05525) (width 0.1) (layer "B.Cu") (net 9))
 (segment (start 150.313017 100.05525) (end 149 100.05525) (width 0.1) (layer "B.Cu") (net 9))
 (segment (start 132.8 103.3) (end 132.8 99.725678) (width 0.1) (layer "F.Cu") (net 2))
 (segment (start 132.8 99.725678) (end 138.285678 94.24) (width 0.1) (layer "F.Cu") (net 2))
 (segment (start 151.428232 104.451) (end 150.33575 104.451) (width 0.1) (layer "F.Cu") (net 2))
 (segment (start 150.33575 104.451) (end 150.3 104.41525) (width 0.1) (layer "F.Cu") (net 2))
 (segment (start 153.668958 96.258624) (end 153.668958 102.210274) (width 0.1) (layer "F.Cu") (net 2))
 (segment (start 151.650334 94.24) (end 153.668958 96.258624) (width 0.1) (layer "F.Cu") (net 2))
 (segment (start 138.285678 94.24) (end 151.650334 94.24) (width 0.1) (layer "F.Cu") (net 2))
 (segment (start 153.668958 102.210274) (end 151.428232 104.451) (width 0.1) (layer "F.Cu") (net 2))
 (via (at 150.3 104.41525) (size 0.6) (drill 0.3) (layers "F.Cu" "B.Cu") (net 2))
 (segment (start 150.215 104.50025) (end 149 104.50025) (width 0.1) (layer "B.Cu") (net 2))
 (segment (start 150.3 104.41525) (end 150.215 104.50025) (width 0.1) (layer "B.Cu") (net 2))
 (segment (start 137.8 98.982458) (end 139.282458 97.5) (width 0.1) (layer "F.Cu") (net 12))
 (segment (start 137.8 103.3) (end 137.8 98.982458) (width 0.1) (layer "F.Cu") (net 12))
 (segment (start 139.282458 97.5) (end 150.3 97.5) (width 0.1) (layer "F.Cu") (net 12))
 (via (at 150.3 97.5) (size 0.6) (drill 0.3) (layers "F.Cu" "B.Cu") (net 12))
 (segment (start 149.64975 98.15025) (end 149 98.15025) (width 0.1) (layer "B.Cu") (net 12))
 (segment (start 150.3 97.5) (end 149.64975 98.15025) (width 0.1) (layer "B.Cu") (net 12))
 (segment (start 145.022471 94.758) (end 147.4282 97.163729) (width 0.1) (layer "B.Cu") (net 14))
 (segment (start 132.3 100.195029) (end 137.737029 94.758) (width 0.1) (layer "B.Cu") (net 14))
 (segment (start 132.3 103.3) (end 132.3 100.195029) (width 0.1) (layer "B.Cu") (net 14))
 (segment (start 147.4282 97.8287) (end 147.74975 98.15025) (width 0.1) (layer "B.Cu") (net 14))
 (segment (start 137.737029 94.758) (end 145.022471 94.758) (width 0.1) (layer "B.Cu") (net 14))
 (segment (start 147.4282 97.163729) (end 147.4282 97.8287) (width 0.1) (layer "B.Cu") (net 14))
 (segment (start 147.74975 98.15025) (end 148.0602 98.15025) (width 0.1) (layer "B.Cu") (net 14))
 (segment (start 146.208 100.3) (end 146.59825 100.69025) (width 0.1) (layer "B.Cu") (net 18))
 (segment (start 146.59825 100.69025) (end 148.0602 100.69025) (width 0.1) (layer "B.Cu") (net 18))
 (segment (start 138.235741 95.962) (end 144.523759 95.962) (width 0.1) (layer "B.Cu") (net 18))
 (segment (start 146.208 97.646241) (end 146.208 100.3) (width 0.1) (layer "B.Cu") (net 18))
 (segment (start 134.3 103.3) (end 134.3 99.897741) (width 0.1) (layer "B.Cu") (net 18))
 (segment (start 134.3 99.897741) (end 138.235741 95.962) (width 0.1) (layer "B.Cu") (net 18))
 (segment (start 144.523759 95.962) (end 146.208 97.646241) (width 0.1) (layer "B.Cu") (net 18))
 (segment (start 151.400978 94.842) (end 153.066958 96.50798) (width 0.1) (layer "F.Cu") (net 4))
 (segment (start 133.8 103.3) (end 133.8 99.577034) (width 0.1) (layer "F.Cu") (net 4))
 (segment (start 153.066958 101.328311) (end 151.195269 103.2) (width 0.1) (layer "F.Cu") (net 4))
 (segment (start 138.535034 94.842) (end 151.400978 94.842) (width 0.1) (layer "F.Cu") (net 4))
 (segment (start 153.066958 96.50798) (end 153.066958 101.328311) (width 0.1) (layer "F.Cu") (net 4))
 (segment (start 151.195269 103.2) (end 150.8 103.2) (width 0.1) (layer "F.Cu") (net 4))
 (segment (start 133.8 99.577034) (end 138.535034 94.842) (width 0.1) (layer "F.Cu") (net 4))
 (via (at 150.8 103.2) (size 0.6) (drill 0.3) (layers "F.Cu" "B.Cu") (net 4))
 (segment (start 150.76975 103.23025) (end 149 103.23025) (width 0.1) (layer "B.Cu") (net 4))
 (segment (start 150.8 103.2) (end 150.76975 103.23025) (width 0.1) (layer "B.Cu") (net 4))
 (segment (start 138.161 93.939) (end 151.775012 93.939) (width 0.1) (layer "F.Cu") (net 1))
 (segment (start 132.3 99.8) (end 138.161 93.939) (width 0.1) (layer "F.Cu") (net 1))
 (segment (start 153.969958 96.133946) (end 153.969958 102.334952) (width 0.1) (layer "F.Cu") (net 1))
 (segment (start 153.969958 102.334952) (end 151.229363 105.075547) (width 0.1) (layer "F.Cu") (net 1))
 (segment (start 151.775012 93.939) (end 153.969958 96.133946) (width 0.1) (layer "F.Cu") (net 1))
 (segment (start 151.229363 105.075547) (end 150.751678 105.075547) (width 0.1) (layer "F.Cu") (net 1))
 (segment (start 132.3 103.3) (end 132.3 99.8) (width 0.1) (layer "F.Cu") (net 1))
 (via (at 150.751678 105.075547) (size 0.6) (drill 0.3) (layers "F.Cu" "B.Cu") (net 1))
 (segment (start 150.691975 105.13525) (end 149 105.13525) (width 0.1) (layer "B.Cu") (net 1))
 (segment (start 150.751678 105.075547) (end 150.691975 105.13525) (width 0.1) (layer "B.Cu") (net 1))
 (segment (start 151.026944 95.745) (end 152.163958 96.882014) (width 0.1) (layer "F.Cu") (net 7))
 (segment (start 152.163958 99.919016) (end 150.735124 101.34785) (width 0.1) (layer "F.Cu") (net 7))
 (segment (start 135.3 99.354068) (end 138.909068 95.745) (width 0.1) (layer "F.Cu") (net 7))
 (segment (start 152.163958 96.882014) (end 152.163958 99.919016) (width 0.1) (layer "F.Cu") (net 7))
 (segment (start 135.3 103.3) (end 135.3 99.354068) (width 0.1) (layer "F.Cu") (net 7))
 (segment (start 138.909068 95.745) (end 151.026944 95.745) (width 0.1) (layer "F.Cu") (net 7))
 (via (at 150.735124 101.34785) (size 0.6) (drill 0.3) (layers "F.Cu" "B.Cu") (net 7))
 (segment (start 150.712524 101.32525) (end 149 101.32525) (width 0.1) (layer "B.Cu") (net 7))
 (segment (start 150.735124 101.34785) (end 150.712524 101.32525) (width 0.1) (layer "B.Cu") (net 7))
 (segment (start 146.93025 99.42025) (end 148.0602 99.42025) (width 0.1) (layer "B.Cu") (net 16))
 (segment (start 137.986385 95.36) (end 144.773115 95.36) (width 0.1) (layer "B.Cu") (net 16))
 (segment (start 146.81 97.396885) (end 146.81 99.3) (width 0.1) (layer "B.Cu") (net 16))
 (segment (start 144.773115 95.36) (end 146.81 97.396885) (width 0.1) (layer "B.Cu") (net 16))
 (segment (start 133.3 100.046385) (end 137.986385 95.36) (width 0.1) (layer "B.Cu") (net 16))
 (segment (start 146.81 99.3) (end 146.93025 99.42025) (width 0.1) (layer "B.Cu") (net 16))
 (segment (start 133.3 103.3) (end 133.3 100.046385) (width 0.1) (layer "B.Cu") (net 16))
 (segment (start 145.907 101.1) (end 146.13225 101.32525) (width 0.1) (layer "B.Cu") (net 19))
 (segment (start 144.399081 96.263) (end 145.907 97.770919) (width 0.1) (layer "B.Cu") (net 19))
 (segment (start 134.8 103.3) (end 134.8 99.823419) (width 0.1) (layer "B.Cu") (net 19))
 (segment (start 138.360419 96.263) (end 144.399081 96.263) (width 0.1) (layer "B.Cu") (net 19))
 (segment (start 145.907 97.770919) (end 145.907 101.1) (width 0.1) (layer "B.Cu") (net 19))
 (segment (start 134.8 99.823419) (end 138.360419 96.263) (width 0.1) (layer "B.Cu") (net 19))
 (segment (start 146.13225 101.32525) (end 148.0602 101.32525) (width 0.1) (layer "B.Cu") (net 19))
 (segment (start 137.3 99.451809) (end 138.983809 97.768) (width 0.1) (layer "B.Cu") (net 24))
 (segment (start 144.402 98.394309) (end 144.402 104.250644) (width 0.1) (layer "B.Cu") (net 24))
 (segment (start 144.651606 104.50025) (end 148.0602 104.50025) (width 0.1) (layer "B.Cu") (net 24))
 (segment (start 138.983809 97.768) (end 143.775691 97.768) (width 0.1) (layer "B.Cu") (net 24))
 (segment (start 137.3 103.3) (end 137.3 99.451809) (width 0.1) (layer "B.Cu") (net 24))
 (segment (start 144.402 104.250644) (end 144.651606 104.50025) (width 0.1) (layer "B.Cu") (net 24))
 (segment (start 143.775691 97.768) (end 144.402 98.394309) (width 0.1) (layer "B.Cu") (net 24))
 (segment (start 144.860928 105.13525) (end 148.0602 105.13525) (width 0.1) (layer "B.Cu") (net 25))
 (segment (start 139.108487 98.069) (end 143.651013 98.069) (width 0.1) (layer "B.Cu") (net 25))
 (segment (start 144.101 104.375322) (end 144.860928 105.13525) (width 0.1) (layer "B.Cu") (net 25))
 (segment (start 137.8 99.377487) (end 139.108487 98.069) (width 0.1) (layer "B.Cu") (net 25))
 (segment (start 144.101 98.518987) (end 144.101 104.375322) (width 0.1) (layer "B.Cu") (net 25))
 (segment (start 143.651013 98.069) (end 144.101 98.518987) (width 0.1) (layer "B.Cu") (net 25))
 (segment (start 137.8 103.3) (end 137.8 99.377487) (width 0.1) (layer "B.Cu") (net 25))
 (segment (start 146.509 99.424678) (end 147.139572 100.05525) (width 0.1) (layer "B.Cu") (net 17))
 (segment (start 138.111063 95.661) (end 144.648437 95.661) (width 0.1) (layer "B.Cu") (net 17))
 (segment (start 146.509 97.521563) (end 146.509 99.424678) (width 0.1) (layer "B.Cu") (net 17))
 (segment (start 133.8 99.972063) (end 138.111063 95.661) (width 0.1) (layer "B.Cu") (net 17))
 (segment (start 133.8 103.3) (end 133.8 99.972063) (width 0.1) (layer "B.Cu") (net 17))
 (segment (start 144.648437 95.661) (end 146.509 97.521563) (width 0.1) (layer "B.Cu") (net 17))
 (segment (start 147.139572 100.05525) (end 148.0602 100.05525) (width 0.1) (layer "B.Cu") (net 17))
 (segment (start 136.8 103.3) (end 136.8 99.526131) (width 0.1) (layer "B.Cu") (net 23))
 (segment (start 144.703 103.403) (end 145.16525 103.86525) (width 0.1) (layer "B.Cu") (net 23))
 (segment (start 145.16525 103.86525) (end 148.0602 103.86525) (width 0.1) (layer "B.Cu") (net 23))
 (segment (start 143.900369 97.467) (end 144.703 98.269631) (width 0.1) (layer "B.Cu") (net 23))
 (segment (start 136.8 99.526131) (end 138.859131 97.467) (width 0.1) (layer "B.Cu") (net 23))
 (segment (start 144.703 98.269631) (end 144.703 103.403) (width 0.1) (layer "B.Cu") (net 23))
 (segment (start 138.859131 97.467) (end 143.900369 97.467) (width 0.1) (layer "B.Cu") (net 23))
 (segment (start 137.861707 95.059) (end 144.897793 95.059) (width 0.1) (layer "B.Cu") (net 15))
 (segment (start 132.8 103.3) (end 132.8 100.120707) (width 0.1) (layer "B.Cu") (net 15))
 (segment (start 147.19625 98.78525) (end 148.0602 98.78525) (width 0.1) (layer "B.Cu") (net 15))
 (segment (start 147.111 97.272207) (end 147.111 98.7) (width 0.1) (layer "B.Cu") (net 15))
 (segment (start 147.111 98.7) (end 147.19625 98.78525) (width 0.1) (layer "B.Cu") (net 15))
 (segment (start 144.897793 95.059) (end 147.111 97.272207) (width 0.1) (layer "B.Cu") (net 15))
 (segment (start 132.8 100.120707) (end 137.861707 95.059) (width 0.1) (layer "B.Cu") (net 15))
 (segment (start 135.3 99.749097) (end 138.485097 96.564) (width 0.1) (layer "B.Cu") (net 20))
 (segment (start 145.606 97.895597) (end 145.606 101.6) (width 0.1) (layer "B.Cu") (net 20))
 (segment (start 138.485097 96.564) (end 144.274403 96.564) (width 0.1) (layer "B.Cu") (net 20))
 (segment (start 145.606 101.6) (end 145.96625 101.96025) (width 0.1) (layer "B.Cu") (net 20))
 (segment (start 144.274403 96.564) (end 145.606 97.895597) (width 0.1) (layer "B.Cu") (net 20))
 (segment (start 145.96625 101.96025) (end 148.0602 101.96025) (width 0.1) (layer "B.Cu") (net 20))
 (segment (start 135.3 103.3) (end 135.3 99.749097) (width 0.1) (layer "B.Cu") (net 20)))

